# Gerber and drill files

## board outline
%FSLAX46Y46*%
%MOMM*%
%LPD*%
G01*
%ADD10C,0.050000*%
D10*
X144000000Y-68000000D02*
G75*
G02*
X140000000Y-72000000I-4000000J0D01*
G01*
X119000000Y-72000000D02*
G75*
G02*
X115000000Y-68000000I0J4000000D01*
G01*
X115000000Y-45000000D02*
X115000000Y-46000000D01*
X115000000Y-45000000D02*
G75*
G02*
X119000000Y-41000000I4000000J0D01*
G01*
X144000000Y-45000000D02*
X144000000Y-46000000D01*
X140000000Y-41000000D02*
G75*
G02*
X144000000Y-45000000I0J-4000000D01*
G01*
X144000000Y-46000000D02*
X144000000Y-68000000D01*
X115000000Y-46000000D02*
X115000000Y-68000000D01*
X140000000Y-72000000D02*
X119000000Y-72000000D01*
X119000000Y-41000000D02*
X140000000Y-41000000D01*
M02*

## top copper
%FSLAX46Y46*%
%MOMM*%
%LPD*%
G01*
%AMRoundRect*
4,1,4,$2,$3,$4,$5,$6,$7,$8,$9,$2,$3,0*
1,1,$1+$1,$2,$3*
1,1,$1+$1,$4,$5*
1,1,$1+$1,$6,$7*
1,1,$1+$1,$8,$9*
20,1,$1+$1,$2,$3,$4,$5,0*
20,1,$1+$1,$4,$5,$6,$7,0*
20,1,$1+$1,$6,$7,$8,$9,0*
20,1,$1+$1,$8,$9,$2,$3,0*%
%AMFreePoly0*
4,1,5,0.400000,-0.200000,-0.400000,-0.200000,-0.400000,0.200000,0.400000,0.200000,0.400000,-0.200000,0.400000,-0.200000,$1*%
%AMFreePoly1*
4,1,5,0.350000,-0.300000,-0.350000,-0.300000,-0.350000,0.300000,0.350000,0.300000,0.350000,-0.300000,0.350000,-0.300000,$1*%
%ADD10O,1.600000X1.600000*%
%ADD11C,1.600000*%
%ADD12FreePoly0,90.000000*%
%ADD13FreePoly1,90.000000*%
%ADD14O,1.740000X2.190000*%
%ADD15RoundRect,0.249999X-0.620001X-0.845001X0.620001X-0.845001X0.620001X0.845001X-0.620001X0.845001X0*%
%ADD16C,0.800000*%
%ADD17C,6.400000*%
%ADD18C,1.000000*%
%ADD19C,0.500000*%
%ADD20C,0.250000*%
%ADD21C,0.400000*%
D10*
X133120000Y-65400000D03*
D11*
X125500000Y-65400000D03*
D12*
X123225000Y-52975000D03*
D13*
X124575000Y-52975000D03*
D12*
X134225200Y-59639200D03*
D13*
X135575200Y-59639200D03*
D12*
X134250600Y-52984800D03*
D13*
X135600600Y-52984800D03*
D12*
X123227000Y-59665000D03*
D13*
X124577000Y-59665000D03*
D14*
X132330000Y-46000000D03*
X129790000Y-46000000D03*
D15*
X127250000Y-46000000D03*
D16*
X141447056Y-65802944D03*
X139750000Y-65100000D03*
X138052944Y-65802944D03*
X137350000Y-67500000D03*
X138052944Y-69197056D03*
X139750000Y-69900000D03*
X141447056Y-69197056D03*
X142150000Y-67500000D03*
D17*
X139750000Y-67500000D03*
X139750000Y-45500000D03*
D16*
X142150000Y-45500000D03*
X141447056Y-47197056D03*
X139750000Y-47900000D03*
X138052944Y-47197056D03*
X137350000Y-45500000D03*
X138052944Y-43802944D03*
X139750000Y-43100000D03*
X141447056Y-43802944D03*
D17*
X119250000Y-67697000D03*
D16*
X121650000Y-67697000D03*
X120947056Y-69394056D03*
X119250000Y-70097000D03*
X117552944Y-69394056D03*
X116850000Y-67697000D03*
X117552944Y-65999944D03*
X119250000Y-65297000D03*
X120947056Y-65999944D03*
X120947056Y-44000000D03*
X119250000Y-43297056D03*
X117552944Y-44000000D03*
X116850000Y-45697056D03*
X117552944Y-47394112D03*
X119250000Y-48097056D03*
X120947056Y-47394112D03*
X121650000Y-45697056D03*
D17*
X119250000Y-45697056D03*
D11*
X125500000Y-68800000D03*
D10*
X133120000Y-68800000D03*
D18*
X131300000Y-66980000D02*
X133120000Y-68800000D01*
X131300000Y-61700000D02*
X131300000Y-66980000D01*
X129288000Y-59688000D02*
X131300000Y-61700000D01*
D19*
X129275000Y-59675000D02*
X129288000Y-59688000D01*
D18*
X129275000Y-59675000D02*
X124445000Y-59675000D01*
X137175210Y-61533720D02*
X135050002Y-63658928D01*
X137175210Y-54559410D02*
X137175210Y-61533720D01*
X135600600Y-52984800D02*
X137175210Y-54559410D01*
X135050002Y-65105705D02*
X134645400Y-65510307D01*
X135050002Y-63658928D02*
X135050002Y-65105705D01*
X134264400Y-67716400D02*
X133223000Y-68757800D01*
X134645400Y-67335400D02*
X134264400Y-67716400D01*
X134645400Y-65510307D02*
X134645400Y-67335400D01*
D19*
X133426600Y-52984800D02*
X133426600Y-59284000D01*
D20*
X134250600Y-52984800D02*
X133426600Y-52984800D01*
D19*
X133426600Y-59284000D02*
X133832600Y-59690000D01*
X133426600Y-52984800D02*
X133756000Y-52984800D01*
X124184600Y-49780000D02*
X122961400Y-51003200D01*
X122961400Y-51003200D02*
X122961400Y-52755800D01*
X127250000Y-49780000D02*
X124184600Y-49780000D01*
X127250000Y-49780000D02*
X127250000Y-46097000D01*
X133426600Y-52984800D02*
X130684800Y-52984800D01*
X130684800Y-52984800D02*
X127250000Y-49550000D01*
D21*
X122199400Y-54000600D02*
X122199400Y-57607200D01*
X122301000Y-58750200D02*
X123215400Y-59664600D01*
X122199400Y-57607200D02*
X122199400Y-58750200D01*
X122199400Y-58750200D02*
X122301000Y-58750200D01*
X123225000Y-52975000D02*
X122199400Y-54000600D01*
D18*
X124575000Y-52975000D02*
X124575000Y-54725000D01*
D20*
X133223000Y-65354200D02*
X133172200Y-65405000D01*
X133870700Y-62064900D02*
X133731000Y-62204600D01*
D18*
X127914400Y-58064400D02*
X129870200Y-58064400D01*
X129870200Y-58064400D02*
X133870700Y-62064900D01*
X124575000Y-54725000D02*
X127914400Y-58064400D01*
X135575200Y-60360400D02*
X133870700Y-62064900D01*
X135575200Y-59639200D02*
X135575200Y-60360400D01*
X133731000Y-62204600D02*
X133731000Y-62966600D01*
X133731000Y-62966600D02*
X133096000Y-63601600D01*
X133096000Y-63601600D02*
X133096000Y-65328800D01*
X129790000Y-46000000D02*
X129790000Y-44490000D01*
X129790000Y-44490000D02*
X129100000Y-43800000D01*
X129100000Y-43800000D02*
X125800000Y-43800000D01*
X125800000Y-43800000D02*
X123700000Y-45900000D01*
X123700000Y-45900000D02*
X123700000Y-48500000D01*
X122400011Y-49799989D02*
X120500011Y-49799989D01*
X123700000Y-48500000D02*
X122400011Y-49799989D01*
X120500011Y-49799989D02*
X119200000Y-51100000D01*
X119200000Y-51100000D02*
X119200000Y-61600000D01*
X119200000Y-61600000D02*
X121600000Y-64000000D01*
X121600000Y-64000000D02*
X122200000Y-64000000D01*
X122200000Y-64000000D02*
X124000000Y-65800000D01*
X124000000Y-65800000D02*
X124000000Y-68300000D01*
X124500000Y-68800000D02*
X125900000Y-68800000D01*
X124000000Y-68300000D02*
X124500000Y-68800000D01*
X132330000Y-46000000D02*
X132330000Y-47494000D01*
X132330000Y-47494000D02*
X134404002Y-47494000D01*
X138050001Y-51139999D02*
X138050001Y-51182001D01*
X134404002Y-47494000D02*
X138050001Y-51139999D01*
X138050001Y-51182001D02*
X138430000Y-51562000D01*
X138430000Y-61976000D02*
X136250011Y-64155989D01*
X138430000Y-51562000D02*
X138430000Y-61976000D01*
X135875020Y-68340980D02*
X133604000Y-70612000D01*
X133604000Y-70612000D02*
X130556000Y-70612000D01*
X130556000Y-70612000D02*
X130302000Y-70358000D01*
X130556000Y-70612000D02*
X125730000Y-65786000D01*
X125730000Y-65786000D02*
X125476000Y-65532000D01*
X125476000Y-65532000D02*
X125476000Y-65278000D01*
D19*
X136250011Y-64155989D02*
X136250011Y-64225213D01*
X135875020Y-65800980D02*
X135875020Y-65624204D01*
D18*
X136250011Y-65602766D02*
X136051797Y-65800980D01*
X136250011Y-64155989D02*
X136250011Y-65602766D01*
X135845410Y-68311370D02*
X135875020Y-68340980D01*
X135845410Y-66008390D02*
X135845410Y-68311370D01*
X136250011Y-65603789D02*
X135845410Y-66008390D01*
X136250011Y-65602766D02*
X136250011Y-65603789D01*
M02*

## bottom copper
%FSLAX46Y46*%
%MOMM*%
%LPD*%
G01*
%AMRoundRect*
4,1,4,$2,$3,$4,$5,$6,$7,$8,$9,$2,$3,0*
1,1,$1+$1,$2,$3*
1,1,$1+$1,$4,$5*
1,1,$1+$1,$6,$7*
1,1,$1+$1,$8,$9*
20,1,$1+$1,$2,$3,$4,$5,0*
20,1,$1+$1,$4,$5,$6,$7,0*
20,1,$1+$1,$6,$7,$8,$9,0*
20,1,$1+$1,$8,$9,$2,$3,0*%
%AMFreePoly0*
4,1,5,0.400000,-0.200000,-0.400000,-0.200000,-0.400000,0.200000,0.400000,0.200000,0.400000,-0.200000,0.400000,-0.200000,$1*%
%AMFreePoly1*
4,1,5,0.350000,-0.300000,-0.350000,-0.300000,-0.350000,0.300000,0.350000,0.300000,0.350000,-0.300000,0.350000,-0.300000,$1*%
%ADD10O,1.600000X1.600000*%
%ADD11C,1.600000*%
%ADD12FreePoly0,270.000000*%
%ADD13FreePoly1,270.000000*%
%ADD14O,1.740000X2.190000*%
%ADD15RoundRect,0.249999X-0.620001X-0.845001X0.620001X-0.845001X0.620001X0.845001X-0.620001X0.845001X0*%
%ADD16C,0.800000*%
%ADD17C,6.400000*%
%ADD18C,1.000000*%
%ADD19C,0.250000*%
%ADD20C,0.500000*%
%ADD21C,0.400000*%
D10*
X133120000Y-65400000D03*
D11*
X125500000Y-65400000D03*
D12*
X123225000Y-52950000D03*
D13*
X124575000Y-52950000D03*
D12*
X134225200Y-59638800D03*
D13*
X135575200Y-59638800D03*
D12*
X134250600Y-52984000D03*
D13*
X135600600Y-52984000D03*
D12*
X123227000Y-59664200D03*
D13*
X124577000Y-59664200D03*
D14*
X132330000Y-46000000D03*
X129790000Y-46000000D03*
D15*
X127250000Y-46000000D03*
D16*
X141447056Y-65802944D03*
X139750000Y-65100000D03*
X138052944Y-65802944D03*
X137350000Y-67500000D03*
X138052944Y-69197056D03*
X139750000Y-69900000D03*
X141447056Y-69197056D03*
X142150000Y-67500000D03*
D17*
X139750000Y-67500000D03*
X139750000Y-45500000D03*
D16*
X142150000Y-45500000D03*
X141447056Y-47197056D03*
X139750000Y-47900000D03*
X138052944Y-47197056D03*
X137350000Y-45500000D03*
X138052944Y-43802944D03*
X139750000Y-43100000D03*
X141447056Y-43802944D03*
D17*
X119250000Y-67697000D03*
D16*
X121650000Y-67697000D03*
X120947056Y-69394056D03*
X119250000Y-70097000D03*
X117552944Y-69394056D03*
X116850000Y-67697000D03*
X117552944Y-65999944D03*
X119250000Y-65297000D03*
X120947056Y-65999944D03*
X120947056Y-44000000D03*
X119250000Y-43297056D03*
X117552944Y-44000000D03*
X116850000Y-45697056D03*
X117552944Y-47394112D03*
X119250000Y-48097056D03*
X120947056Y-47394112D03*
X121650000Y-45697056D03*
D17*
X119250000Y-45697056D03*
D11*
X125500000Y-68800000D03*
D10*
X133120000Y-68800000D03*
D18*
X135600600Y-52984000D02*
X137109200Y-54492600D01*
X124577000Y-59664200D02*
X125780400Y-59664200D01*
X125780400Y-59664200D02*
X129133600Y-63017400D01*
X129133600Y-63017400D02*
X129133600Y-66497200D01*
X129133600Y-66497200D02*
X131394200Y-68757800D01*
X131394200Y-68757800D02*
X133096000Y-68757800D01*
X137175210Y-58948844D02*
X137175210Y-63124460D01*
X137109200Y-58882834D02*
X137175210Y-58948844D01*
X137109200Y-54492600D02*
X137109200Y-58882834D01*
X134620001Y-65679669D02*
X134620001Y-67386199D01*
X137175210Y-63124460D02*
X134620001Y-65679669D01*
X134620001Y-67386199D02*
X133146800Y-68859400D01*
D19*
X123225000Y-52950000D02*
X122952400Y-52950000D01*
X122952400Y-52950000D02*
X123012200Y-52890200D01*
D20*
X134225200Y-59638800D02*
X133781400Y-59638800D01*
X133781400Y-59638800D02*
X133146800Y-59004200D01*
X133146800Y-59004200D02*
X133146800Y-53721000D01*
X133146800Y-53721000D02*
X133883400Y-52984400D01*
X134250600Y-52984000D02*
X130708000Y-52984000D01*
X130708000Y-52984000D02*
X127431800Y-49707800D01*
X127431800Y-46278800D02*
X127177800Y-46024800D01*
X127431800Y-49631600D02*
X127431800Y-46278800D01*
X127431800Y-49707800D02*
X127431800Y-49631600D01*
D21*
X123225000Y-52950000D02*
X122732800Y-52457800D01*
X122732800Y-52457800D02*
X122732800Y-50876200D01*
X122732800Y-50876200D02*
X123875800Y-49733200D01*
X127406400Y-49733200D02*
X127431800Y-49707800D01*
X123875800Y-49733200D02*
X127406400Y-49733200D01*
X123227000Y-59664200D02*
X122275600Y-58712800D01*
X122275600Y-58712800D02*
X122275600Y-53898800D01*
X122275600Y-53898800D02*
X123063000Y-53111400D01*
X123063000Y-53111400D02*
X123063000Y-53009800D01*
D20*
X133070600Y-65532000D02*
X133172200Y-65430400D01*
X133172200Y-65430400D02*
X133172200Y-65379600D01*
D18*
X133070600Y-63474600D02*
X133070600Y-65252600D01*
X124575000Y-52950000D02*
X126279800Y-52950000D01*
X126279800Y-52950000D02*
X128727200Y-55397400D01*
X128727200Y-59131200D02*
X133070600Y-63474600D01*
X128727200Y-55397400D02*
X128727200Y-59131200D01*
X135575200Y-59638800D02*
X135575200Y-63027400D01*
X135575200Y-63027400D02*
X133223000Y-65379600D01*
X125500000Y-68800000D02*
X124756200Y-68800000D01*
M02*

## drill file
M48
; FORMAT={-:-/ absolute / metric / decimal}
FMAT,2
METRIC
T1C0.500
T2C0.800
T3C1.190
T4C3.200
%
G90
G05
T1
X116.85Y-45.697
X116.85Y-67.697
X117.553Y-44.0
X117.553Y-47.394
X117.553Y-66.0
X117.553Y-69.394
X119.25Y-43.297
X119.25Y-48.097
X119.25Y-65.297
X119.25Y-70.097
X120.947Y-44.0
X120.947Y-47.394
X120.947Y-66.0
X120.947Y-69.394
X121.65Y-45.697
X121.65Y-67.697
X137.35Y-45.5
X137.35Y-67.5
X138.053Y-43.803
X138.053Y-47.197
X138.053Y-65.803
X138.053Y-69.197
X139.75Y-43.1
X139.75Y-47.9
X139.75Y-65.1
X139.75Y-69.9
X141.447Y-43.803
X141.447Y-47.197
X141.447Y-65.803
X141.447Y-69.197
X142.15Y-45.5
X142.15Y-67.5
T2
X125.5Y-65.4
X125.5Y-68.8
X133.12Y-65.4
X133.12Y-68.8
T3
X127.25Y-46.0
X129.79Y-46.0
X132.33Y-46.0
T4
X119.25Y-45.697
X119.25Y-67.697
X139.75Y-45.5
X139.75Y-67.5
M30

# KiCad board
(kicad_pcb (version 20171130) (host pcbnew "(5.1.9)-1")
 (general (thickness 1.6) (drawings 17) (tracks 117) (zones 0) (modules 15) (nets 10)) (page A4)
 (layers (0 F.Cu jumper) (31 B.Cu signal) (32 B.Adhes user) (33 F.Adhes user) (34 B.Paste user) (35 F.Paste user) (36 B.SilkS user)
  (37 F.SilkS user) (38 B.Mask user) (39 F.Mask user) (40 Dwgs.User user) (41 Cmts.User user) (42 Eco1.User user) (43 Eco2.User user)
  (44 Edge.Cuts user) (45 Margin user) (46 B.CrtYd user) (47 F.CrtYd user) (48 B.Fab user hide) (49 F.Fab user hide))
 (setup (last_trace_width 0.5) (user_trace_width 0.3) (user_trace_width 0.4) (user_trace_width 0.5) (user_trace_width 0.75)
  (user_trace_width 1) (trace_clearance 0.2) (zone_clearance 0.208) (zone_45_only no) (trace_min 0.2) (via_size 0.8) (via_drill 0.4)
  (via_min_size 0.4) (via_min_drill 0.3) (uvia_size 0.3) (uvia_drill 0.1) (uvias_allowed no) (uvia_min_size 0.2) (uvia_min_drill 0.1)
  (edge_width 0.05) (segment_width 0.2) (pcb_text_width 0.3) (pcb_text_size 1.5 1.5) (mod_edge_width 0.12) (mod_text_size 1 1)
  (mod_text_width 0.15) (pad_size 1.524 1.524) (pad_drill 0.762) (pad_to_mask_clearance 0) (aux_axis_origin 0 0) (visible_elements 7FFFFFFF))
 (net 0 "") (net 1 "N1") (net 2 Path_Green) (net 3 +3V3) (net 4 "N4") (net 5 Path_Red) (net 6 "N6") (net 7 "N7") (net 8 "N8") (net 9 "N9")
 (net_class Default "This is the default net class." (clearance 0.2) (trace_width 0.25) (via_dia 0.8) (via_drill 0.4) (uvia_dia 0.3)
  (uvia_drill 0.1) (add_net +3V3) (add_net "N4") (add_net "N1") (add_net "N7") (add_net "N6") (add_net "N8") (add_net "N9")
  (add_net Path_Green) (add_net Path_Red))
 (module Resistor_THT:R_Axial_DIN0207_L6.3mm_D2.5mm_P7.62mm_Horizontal (layer F.Cu) (at 125.5 65.4)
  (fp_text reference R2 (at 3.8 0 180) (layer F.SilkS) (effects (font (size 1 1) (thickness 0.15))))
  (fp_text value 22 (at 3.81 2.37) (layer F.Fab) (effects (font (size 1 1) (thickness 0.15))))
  (pad 2 thru_hole oval (at 7.62 0) (size 1.6 1.6) (drill 0.8) (layers *.Cu *.Mask) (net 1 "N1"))
  (pad 1 thru_hole circle (at 0 0) (size 1.6 1.6) (drill 0.8) (layers *.Cu *.Mask) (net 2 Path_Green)))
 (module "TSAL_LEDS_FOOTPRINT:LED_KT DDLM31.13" (layer F.Cu) (at 123.95 53 90)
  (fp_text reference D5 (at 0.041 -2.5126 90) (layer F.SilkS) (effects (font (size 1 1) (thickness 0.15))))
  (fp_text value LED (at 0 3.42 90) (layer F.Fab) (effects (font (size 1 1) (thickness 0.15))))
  (pad 2 smd custom (at 0.025 -0.725 90) (size 0.8 0.4) (layers F.Cu F.Paste F.Mask) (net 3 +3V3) (zone_connect 0)
   (options (clearance outline) (anchor rect)) (primitives))
  (pad 1 smd custom (at 0.025 0.625 90) (size 0.7 0.6) (layers F.Cu F.Paste F.Mask) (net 1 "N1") (zone_connect 0)
   (options (clearance outline) (anchor rect)) (primitives)))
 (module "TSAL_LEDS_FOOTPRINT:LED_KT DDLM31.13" (layer B.Cu) (at 123.95 52.925 270)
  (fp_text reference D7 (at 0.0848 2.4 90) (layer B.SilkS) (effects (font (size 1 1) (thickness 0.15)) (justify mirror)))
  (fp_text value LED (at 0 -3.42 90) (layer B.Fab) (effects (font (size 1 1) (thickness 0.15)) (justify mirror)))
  (pad 2 smd custom (at 0.025 0.725 270) (size 0.8 0.4) (layers B.Cu B.Paste B.Mask) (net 3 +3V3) (zone_connect 0)
   (options (clearance outline) (anchor rect)) (primitives))
  (pad 1 smd custom (at 0.025 -0.625 270) (size 0.7 0.6) (layers B.Cu B.Paste B.Mask) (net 1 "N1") (zone_connect 0)
   (options (clearance outline) (anchor rect)) (primitives)))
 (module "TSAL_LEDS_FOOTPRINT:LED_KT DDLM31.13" (layer B.Cu) (at 134.9502 59.6138 270)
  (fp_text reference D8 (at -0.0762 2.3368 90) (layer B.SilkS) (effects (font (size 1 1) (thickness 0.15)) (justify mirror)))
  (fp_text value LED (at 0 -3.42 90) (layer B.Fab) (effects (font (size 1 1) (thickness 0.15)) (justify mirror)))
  (pad 2 smd custom (at 0.025 0.725 270) (size 0.8 0.4) (layers B.Cu B.Paste B.Mask) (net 3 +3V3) (zone_connect 0)
   (options (clearance outline) (anchor rect)) (primitives))
  (pad 1 smd custom (at 0.025 -0.625 270) (size 0.7 0.6) (layers B.Cu B.Paste B.Mask) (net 1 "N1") (zone_connect 0)
   (options (clearance outline) (anchor rect)) (primitives)))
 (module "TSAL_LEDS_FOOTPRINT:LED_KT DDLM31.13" (layer F.Cu) (at 134.9502 59.6642 90)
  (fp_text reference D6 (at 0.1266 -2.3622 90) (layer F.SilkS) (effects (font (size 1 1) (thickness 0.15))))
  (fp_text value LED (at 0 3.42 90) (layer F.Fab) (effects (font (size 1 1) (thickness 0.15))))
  (pad 2 smd custom (at 0.025 -0.725 90) (size 0.8 0.4) (layers F.Cu F.Paste F.Mask) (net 3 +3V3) (zone_connect 0)
   (options (clearance outline) (anchor rect)) (primitives))
  (pad 1 smd custom (at 0.025 0.625 90) (size 0.7 0.6) (layers F.Cu F.Paste F.Mask) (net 1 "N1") (zone_connect 0)
   (options (clearance outline) (anchor rect)) (primitives)))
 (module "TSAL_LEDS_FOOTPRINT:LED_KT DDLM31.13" (layer B.Cu) (at 134.9756 52.959 270)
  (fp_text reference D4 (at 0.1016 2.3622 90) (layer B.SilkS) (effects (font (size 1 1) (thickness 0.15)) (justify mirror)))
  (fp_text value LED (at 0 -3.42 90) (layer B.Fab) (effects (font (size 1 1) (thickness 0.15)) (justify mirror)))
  (pad 2 smd custom (at 0.025 0.725 270) (size 0.8 0.4) (layers B.Cu B.Paste B.Mask) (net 3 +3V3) (zone_connect 0)
   (options (clearance outline) (anchor rect)) (primitives))
  (pad 1 smd custom (at 0.025 -0.625 270) (size 0.7 0.6) (layers B.Cu B.Paste B.Mask) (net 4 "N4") (zone_connect 0)
   (options (clearance outline) (anchor rect)) (primitives)))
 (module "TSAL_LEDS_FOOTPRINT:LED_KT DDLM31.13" (layer B.Cu) (at 123.952 59.6392 270)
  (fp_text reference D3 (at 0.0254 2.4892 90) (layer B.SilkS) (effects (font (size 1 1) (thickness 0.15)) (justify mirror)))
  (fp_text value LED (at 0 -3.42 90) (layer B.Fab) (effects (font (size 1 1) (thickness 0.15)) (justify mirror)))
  (pad 2 smd custom (at 0.025 0.725 270) (size 0.8 0.4) (layers B.Cu B.Paste B.Mask) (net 3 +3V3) (zone_connect 0)
   (options (clearance outline) (anchor rect)) (primitives))
  (pad 1 smd custom (at 0.025 -0.625 270) (size 0.7 0.6) (layers B.Cu B.Paste B.Mask) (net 4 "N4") (zone_connect 0)
   (options (clearance outline) (anchor rect)) (primitives)))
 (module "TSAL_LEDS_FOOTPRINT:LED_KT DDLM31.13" (layer F.Cu) (at 134.9756 53.0098 90)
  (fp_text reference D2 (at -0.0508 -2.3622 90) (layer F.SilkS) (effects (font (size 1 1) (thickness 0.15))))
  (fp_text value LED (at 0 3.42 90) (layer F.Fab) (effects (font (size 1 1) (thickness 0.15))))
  (pad 2 smd custom (at 0.025 -0.725 90) (size 0.8 0.4) (layers F.Cu F.Paste F.Mask) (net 3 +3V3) (zone_connect 0)
   (options (clearance outline) (anchor rect)) (primitives))
  (pad 1 smd custom (at 0.025 0.625 90) (size 0.7 0.6) (layers F.Cu F.Paste F.Mask) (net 4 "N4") (zone_connect 0)
   (options (clearance outline) (anchor rect)) (primitives)))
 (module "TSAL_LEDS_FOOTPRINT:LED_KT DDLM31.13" (layer F.Cu) (at 123.952 59.69 90)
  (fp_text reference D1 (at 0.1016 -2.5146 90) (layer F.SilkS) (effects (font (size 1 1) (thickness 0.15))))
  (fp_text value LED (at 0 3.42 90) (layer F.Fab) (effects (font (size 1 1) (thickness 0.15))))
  (pad 2 smd custom (at 0.025 -0.725 90) (size 0.8 0.4) (layers F.Cu F.Paste F.Mask) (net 3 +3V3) (zone_connect 0)
   (options (clearance outline) (anchor rect)) (primitives))
  (pad 1 smd custom (at 0.025 0.625 90) (size 0.7 0.6) (layers F.Cu F.Paste F.Mask) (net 4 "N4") (zone_connect 0)
   (options (clearance outline) (anchor rect)) (primitives)))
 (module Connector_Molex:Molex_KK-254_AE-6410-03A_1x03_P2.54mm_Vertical (layer F.Cu) (at 127.25 46)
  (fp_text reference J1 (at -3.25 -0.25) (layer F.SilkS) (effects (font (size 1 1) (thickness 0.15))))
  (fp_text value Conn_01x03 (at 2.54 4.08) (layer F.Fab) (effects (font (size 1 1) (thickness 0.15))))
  (pad 3 thru_hole oval (at 5.08 0) (size 1.74 2.19) (drill 1.19) (layers *.Cu *.Mask) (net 2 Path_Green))
  (pad 2 thru_hole oval (at 2.54 0) (size 1.74 2.19) (drill 1.19) (layers *.Cu *.Mask) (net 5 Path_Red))
  (pad 1 thru_hole roundrect (at 0 0) (size 1.74 2.19) (drill 1.19) (layers *.Cu *.Mask) (roundrect_rratio 0.1436775862068966) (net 3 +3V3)))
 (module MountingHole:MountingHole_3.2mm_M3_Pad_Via (layer F.Cu) (at 139.75 67.5)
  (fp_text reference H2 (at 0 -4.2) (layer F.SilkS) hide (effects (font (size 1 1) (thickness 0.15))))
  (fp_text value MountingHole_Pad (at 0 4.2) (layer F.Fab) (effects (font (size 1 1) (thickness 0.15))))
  (pad 1 thru_hole circle (at 1.697056 -1.697056) (size 0.8 0.8) (drill 0.5) (layers *.Cu *.Mask) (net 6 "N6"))
  (pad 1 thru_hole circle (at 0 -2.4) (size 0.8 0.8) (drill 0.5) (layers *.Cu *.Mask) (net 6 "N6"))
  (pad 1 thru_hole circle (at -1.697056 -1.697056) (size 0.8 0.8) (drill 0.5) (layers *.Cu *.Mask) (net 6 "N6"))
  (pad 1 thru_hole circle (at -2.4 0) (size 0.8 0.8) (drill 0.5) (layers *.Cu *.Mask) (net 6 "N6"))
  (pad 1 thru_hole circle (at -1.697056 1.697056) (size 0.8 0.8) (drill 0.5) (layers *.Cu *.Mask) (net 6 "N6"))
  (pad 1 thru_hole circle (at 0 2.4) (size 0.8 0.8) (drill 0.5) (layers *.Cu *.Mask) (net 6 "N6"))
  (pad 1 thru_hole circle (at 1.697056 1.697056) (size 0.8 0.8) (drill 0.5) (layers *.Cu *.Mask) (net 6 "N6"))
  (pad 1 thru_hole circle (at 2.4 0) (size 0.8 0.8) (drill 0.5) (layers *.Cu *.Mask) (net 6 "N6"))
  (pad 1 thru_hole circle (at 0 0) (size 6.4 6.4) (drill 3.2) (layers *.Cu *.Mask) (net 6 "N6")))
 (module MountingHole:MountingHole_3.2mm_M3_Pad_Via (layer F.Cu) (at 139.75 45.5)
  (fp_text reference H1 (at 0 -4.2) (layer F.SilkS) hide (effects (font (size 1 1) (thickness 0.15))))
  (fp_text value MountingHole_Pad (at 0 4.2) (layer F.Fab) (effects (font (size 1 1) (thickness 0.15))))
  (pad 1 thru_hole circle (at 0 0) (size 6.4 6.4) (drill 3.2) (layers *.Cu *.Mask) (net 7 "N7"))
  (pad 1 thru_hole circle (at 2.4 0) (size 0.8 0.8) (drill 0.5) (layers *.Cu *.Mask) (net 7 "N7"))
  (pad 1 thru_hole circle (at 1.697056 1.697056) (size 0.8 0.8) (drill 0.5) (layers *.Cu *.Mask) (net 7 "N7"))
  (pad 1 thru_hole circle (at 0 2.4) (size 0.8 0.8) (drill 0.5) (layers *.Cu *.Mask) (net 7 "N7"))
  (pad 1 thru_hole circle (at -1.697056 1.697056) (size 0.8 0.8) (drill 0.5) (layers *.Cu *.Mask) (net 7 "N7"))
  (pad 1 thru_hole circle (at -2.4 0) (size 0.8 0.8) (drill 0.5) (layers *.Cu *.Mask) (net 7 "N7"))
  (pad 1 thru_hole circle (at -1.697056 -1.697056) (size 0.8 0.8) (drill 0.5) (layers *.Cu *.Mask) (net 7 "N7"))
  (pad 1 thru_hole circle (at 0 -2.4) (size 0.8 0.8) (drill 0.5) (layers *.Cu *.Mask) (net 7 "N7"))
  (pad 1 thru_hole circle (at 1.697056 -1.697056) (size 0.8 0.8) (drill 0.5) (layers *.Cu *.Mask) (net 7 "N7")))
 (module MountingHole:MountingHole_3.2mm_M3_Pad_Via (layer F.Cu) (at 119.25 67.697)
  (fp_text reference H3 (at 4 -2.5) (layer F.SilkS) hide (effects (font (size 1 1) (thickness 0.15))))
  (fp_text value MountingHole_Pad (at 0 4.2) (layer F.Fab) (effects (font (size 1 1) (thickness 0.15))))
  (pad 1 thru_hole circle (at 0 0) (size 6.4 6.4) (drill 3.2) (layers *.Cu *.Mask) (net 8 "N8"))
  (pad 1 thru_hole circle (at 2.4 0) (size 0.8 0.8) (drill 0.5) (layers *.Cu *.Mask) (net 8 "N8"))
  (pad 1 thru_hole circle (at 1.697056 1.697056) (size 0.8 0.8) (drill 0.5) (layers *.Cu *.Mask) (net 8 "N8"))
  (pad 1 thru_hole circle (at 0 2.4) (size 0.8 0.8) (drill 0.5) (layers *.Cu *.Mask) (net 8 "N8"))
  (pad 1 thru_hole circle (at -1.697056 1.697056) (size 0.8 0.8) (drill 0.5) (layers *.Cu *.Mask) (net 8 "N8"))
  (pad 1 thru_hole circle (at -2.4 0) (size 0.8 0.8) (drill 0.5) (layers *.Cu *.Mask) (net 8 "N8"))
  (pad 1 thru_hole circle (at -1.697056 -1.697056) (size 0.8 0.8) (drill 0.5) (layers *.Cu *.Mask) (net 8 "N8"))
  (pad 1 thru_hole circle (at 0 -2.4) (size 0.8 0.8) (drill 0.5) (layers *.Cu *.Mask) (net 8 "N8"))
  (pad 1 thru_hole circle (at 1.697056 -1.697056) (size 0.8 0.8) (drill 0.5) (layers *.Cu *.Mask) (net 8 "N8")))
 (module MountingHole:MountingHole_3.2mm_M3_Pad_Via (layer F.Cu) (at 119.25 45.697056)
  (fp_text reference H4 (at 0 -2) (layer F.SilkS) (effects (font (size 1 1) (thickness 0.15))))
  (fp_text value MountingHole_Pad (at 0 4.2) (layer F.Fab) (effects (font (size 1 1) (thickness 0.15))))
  (pad 1 thru_hole circle (at 1.697056 -1.697056) (size 0.8 0.8) (drill 0.5) (layers *.Cu *.Mask) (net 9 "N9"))
  (pad 1 thru_hole circle (at 0 -2.4) (size 0.8 0.8) (drill 0.5) (layers *.Cu *.Mask) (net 9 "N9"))
  (pad 1 thru_hole circle (at -1.697056 -1.697056) (size 0.8 0.8) (drill 0.5) (layers *.Cu *.Mask) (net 9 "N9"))
  (pad 1 thru_hole circle (at -2.4 0) (size 0.8 0.8) (drill 0.5) (layers *.Cu *.Mask) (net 9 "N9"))
  (pad 1 thru_hole circle (at -1.697056 1.697056) (size 0.8 0.8) (drill 0.5) (layers *.Cu *.Mask) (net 9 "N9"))
  (pad 1 thru_hole circle (at 0 2.4) (size 0.8 0.8) (drill 0.5) (layers *.Cu *.Mask) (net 9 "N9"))
  (pad 1 thru_hole circle (at 1.697056 1.697056) (size 0.8 0.8) (drill 0.5) (layers *.Cu *.Mask) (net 9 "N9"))
  (pad 1 thru_hole circle (at 2.4 0) (size 0.8 0.8) (drill 0.5) (layers *.Cu *.Mask) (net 9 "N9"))
  (pad 1 thru_hole circle (at 0 0) (size 6.4 6.4) (drill 3.2) (layers *.Cu *.Mask) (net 9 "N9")))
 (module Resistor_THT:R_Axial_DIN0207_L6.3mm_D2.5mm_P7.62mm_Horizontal (layer F.Cu) (at 125.5 68.8)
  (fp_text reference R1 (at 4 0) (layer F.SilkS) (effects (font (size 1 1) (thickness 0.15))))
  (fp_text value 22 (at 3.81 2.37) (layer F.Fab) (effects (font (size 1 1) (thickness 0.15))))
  (pad 1 thru_hole circle (at 0 0) (size 1.6 1.6) (drill 0.8) (layers *.Cu *.Mask) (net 5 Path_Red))
  (pad 2 thru_hole oval (at 7.62 0) (size 1.6 1.6) (drill 0.8) (layers *.Cu *.Mask) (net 4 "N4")))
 (gr_arc (start 140 68) (end 140 72) (angle -90) (layer Edge.Cuts) (width 0.05))
 (gr_arc (start 119 68) (end 115 68) (angle -90) (layer Edge.Cuts) (width 0.05))
 (gr_line (start 115 45) (end 115 46) (layer Edge.Cuts) (width 0.05))
 (gr_arc (start 119 45) (end 119 41) (angle -90) (layer Edge.Cuts) (width 0.05))
 (gr_line (start 144 45) (end 144 46) (layer Edge.Cuts) (width 0.05))
 (gr_arc (start 140 45) (end 144 45) (angle -90) (layer Edge.Cuts) (width 0.05))
 (gr_line (start 144 46) (end 144 68) (layer Edge.Cuts) (width 0.05))
 (gr_line (start 115 46) (end 115 68) (layer Edge.Cuts) (width 0.05))
 (gr_line (start 140 72) (end 119 72) (layer Edge.Cuts) (width 0.05))
 (gr_line (start 119 41) (end 140 41) (layer Edge.Cuts) (width 0.05))
 (segment (start 131.3 66.98) (end 133.12 68.8) (width 1) (layer F.Cu) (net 4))
 (segment (start 131.3 61.7) (end 131.3 66.98) (width 1) (layer F.Cu) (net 4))
 (segment (start 129.288 59.688) (end 131.3 61.7) (width 1) (layer F.Cu) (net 4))
 (segment (start 129.275 59.675) (end 129.288 59.688) (width 0.5) (layer F.Cu) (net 4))
 (segment (start 129.275 59.675) (end 124.445 59.675) (width 1) (layer F.Cu) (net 4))
 (segment (start 137.17521 61.53372) (end 135.050002 63.658928) (width 1) (layer F.Cu) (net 4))
 (segment (start 137.17521 54.55941) (end 137.17521 61.53372) (width 1) (layer F.Cu) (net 4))
 (segment (start 135.6006 52.9848) (end 137.17521 54.55941) (width 1) (layer F.Cu) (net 4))
 (segment (start 135.050002 65.105705) (end 134.6454 65.510307) (width 1) (layer F.Cu) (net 4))
 (segment (start 135.050002 63.658928) (end 135.050002 65.105705) (width 1) (layer F.Cu) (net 4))
 (segment (start 134.2644 67.7164) (end 133.223 68.7578) (width 1) (layer F.Cu) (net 4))
 (segment (start 135.6006 52.984) (end 137.1092 54.4926) (width 1) (layer B.Cu) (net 4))
 (segment (start 124.577 59.6642) (end 125.7804 59.6642) (width 1) (layer B.Cu) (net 4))
 (segment (start 125.7804 59.6642) (end 129.1336 63.0174) (width 1) (layer B.Cu) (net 4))
 (segment (start 129.1336 63.0174) (end 129.1336 66.4972) (width 1) (layer B.Cu) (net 4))
 (segment (start 129.1336 66.4972) (end 131.3942 68.7578) (width 1) (layer B.Cu) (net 4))
 (segment (start 131.3942 68.7578) (end 133.096 68.7578) (width 1) (layer B.Cu) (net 4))
 (segment (start 134.6454 67.3354) (end 134.2644 67.7164) (width 1) (layer F.Cu) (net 4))
 (segment (start 134.6454 65.510307) (end 134.6454 67.3354) (width 1) (layer F.Cu) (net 4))
 (segment (start 137.17521 58.948844) (end 137.17521 63.12446) (width 1) (layer B.Cu) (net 4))
 (segment (start 137.1092 58.882834) (end 137.17521 58.948844) (width 1) (layer B.Cu) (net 4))
 (segment (start 137.1092 54.4926) (end 137.1092 58.882834) (width 1) (layer B.Cu) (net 4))
 (segment (start 134.620001 65.679669) (end 134.620001 67.386199) (width 1) (layer B.Cu) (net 4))
 (segment (start 137.17521 63.12446) (end 134.620001 65.679669) (width 1) (layer B.Cu) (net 4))
 (segment (start 134.620001 67.386199) (end 133.1468 68.8594) (width 1) (layer B.Cu) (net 4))
 (segment (start 123.225 52.95) (end 122.9524 52.95) (width 0.25) (layer B.Cu) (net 3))
 (segment (start 122.9524 52.95) (end 123.0122 52.8902) (width 0.25) (layer B.Cu) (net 3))
 (segment (start 133.4266 52.9848) (end 133.4266 59.284) (width 0.5) (layer F.Cu) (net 3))
 (segment (start 134.2506 52.9848) (end 133.4266 52.9848) (width 0.25) (layer F.Cu) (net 3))
 (segment (start 133.4266 59.284) (end 133.8326 59.69) (width 0.5) (layer F.Cu) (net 3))
 (segment (start 133.4266 52.9848) (end 133.756 52.9848) (width 0.5) (layer F.Cu) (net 3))
 (segment (start 124.1846 49.78) (end 122.9614 51.0032) (width 0.5) (layer F.Cu) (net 3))
 (segment (start 122.9614 51.0032) (end 122.9614 52.7558) (width 0.5) (layer F.Cu) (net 3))
 (segment (start 127.25 49.78) (end 124.1846 49.78) (width 0.5) (layer F.Cu) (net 3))
 (segment (start 127.25 49.78) (end 127.25 46.097) (width 0.5) (layer F.Cu) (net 3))
 (segment (start 134.2252 59.6388) (end 133.7814 59.6388) (width 0.5) (layer B.Cu) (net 3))
 (segment (start 133.7814 59.6388) (end 133.1468 59.0042) (width 0.5) (layer B.Cu) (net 3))
 (segment (start 133.1468 59.0042) (end 133.1468 53.721) (width 0.5) (layer B.Cu) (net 3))
 (segment (start 133.1468 53.721) (end 133.8834 52.9844) (width 0.5) (layer B.Cu) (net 3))
 (segment (start 133.4266 52.9848) (end 130.6848 52.9848) (width 0.5) (layer F.Cu) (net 3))
 (segment (start 130.6848 52.9848) (end 127.25 49.55) (width 0.5) (layer F.Cu) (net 3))
 (segment (start 134.2506 52.984) (end 130.708 52.984) (width 0.5) (layer B.Cu) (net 3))
 (segment (start 130.708 52.984) (end 127.4318 49.7078) (width 0.5) (layer B.Cu) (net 3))
 (segment (start 127.4318 46.2788) (end 127.1778 46.0248) (width 0.5) (layer B.Cu) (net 3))
 (segment (start 127.4318 49.6316) (end 127.4318 46.2788) (width 0.5) (layer B.Cu) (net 3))
 (segment (start 127.4318 49.7078) (end 127.4318 49.6316) (width 0.5) (layer B.Cu) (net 3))
 (segment (start 123.225 52.95) (end 122.7328 52.4578) (width 0.4) (layer B.Cu) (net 3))
 (segment (start 122.7328 52.4578) (end 122.7328 50.8762) (width 0.4) (layer B.Cu) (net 3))
 (segment (start 122.7328 50.8762) (end 123.8758 49.7332) (width 0.4) (layer B.Cu) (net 3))
 (segment (start 127.4064 49.7332) (end 127.4318 49.7078) (width 0.4) (layer B.Cu) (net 3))
 (segment (start 123.8758 49.7332) (end 127.4064 49.7332) (width 0.4) (layer B.Cu) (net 3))
 (segment (start 122.1994 54.0006) (end 122.1994 57.6072) (width 0.4) (layer F.Cu) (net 3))
 (segment (start 122.301 58.7502) (end 123.2154 59.6646) (width 0.4) (layer F.Cu) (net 3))
 (segment (start 122.1994 57.6072) (end 122.1994 58.7502) (width 0.4) (layer F.Cu) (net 3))
 (segment (start 122.1994 58.7502) (end 122.301 58.7502) (width 0.4) (layer F.Cu) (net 3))
 (segment (start 123.225 52.975) (end 122.1994 54.0006) (width 0.4) (layer F.Cu) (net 3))
 (segment (start 123.227 59.6642) (end 122.2756 58.7128) (width 0.4) (layer B.Cu) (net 3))
 (segment (start 122.2756 58.7128) (end 122.2756 53.8988) (width 0.4) (layer B.Cu) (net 3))
 (segment (start 122.2756 53.8988) (end 123.063 53.1114) (width 0.4) (layer B.Cu) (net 3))
 (segment (start 123.063 53.1114) (end 123.063 53.0098) (width 0.4) (layer B.Cu) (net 3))
 (segment (start 133.0706 65.532) (end 133.1722 65.4304) (width 0.5) (layer B.Cu) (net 1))
 (segment (start 133.1722 65.4304) (end 133.1722 65.3796) (width 0.5) (layer B.Cu) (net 1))
 (segment (start 124.575 52.975) (end 124.575 54.725) (width 1) (layer F.Cu) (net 1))
 (segment (start 133.223 65.3542) (end 133.1722 65.405) (width 0.25) (layer F.Cu) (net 1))
 (segment (start 133.8707 62.0649) (end 133.731 62.2046) (width 0.25) (layer F.Cu) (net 1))
 (segment (start 127.9144 58.0644) (end 129.8702 58.0644) (width 1) (layer F.Cu) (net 1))
 (segment (start 129.8702 58.0644) (end 133.8707 62.0649) (width 1) (layer F.Cu) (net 1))
 (segment (start 124.575 54.725) (end 127.9144 58.0644) (width 1) (layer F.Cu) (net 1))
 (segment (start 135.5752 60.3604) (end 133.8707 62.0649) (width 1) (layer F.Cu) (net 1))
 (segment (start 135.5752 59.6392) (end 135.5752 60.3604) (width 1) (layer F.Cu) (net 1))
 (segment (start 133.731 62.2046) (end 133.731 62.9666) (width 1) (layer F.Cu) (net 1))
 (segment (start 133.731 62.9666) (end 133.096 63.6016) (width 1) (layer F.Cu) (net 1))
 (segment (start 133.096 63.6016) (end 133.096 65.3288) (width 1) (layer F.Cu) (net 1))
 (segment (start 133.0706 63.4746) (end 133.0706 65.2526) (width 1) (layer B.Cu) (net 1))
 (segment (start 124.575 52.95) (end 126.2798 52.95) (width 1) (layer B.Cu) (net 1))
 (segment (start 126.2798 52.95) (end 128.7272 55.3974) (width 1) (layer B.Cu) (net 1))
 (segment (start 128.7272 59.1312) (end 133.0706 63.4746) (width 1) (layer B.Cu) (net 1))
 (segment (start 128.7272 55.3974) (end 128.7272 59.1312) (width 1) (layer B.Cu) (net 1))
 (segment (start 135.5752 59.6388) (end 135.5752 63.0274) (width 1) (layer B.Cu) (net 1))
 (segment (start 135.5752 63.0274) (end 133.223 65.3796) (width 1) (layer B.Cu) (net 1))
 (segment (start 129.79 46) (end 129.79 44.49) (width 1) (layer F.Cu) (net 5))
 (segment (start 129.79 44.49) (end 129.1 43.8) (width 1) (layer F.Cu) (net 5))
 (segment (start 129.1 43.8) (end 125.8 43.8) (width 1) (layer F.Cu) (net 5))
 (segment (start 125.8 43.8) (end 123.7 45.9) (width 1) (layer F.Cu) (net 5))
 (segment (start 123.7 45.9) (end 123.7 48.5) (width 1) (layer F.Cu) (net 5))
 (segment (start 122.400011 49.799989) (end 120.500011 49.799989) (width 1) (layer F.Cu) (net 5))
 (segment (start 123.7 48.5) (end 122.400011 49.799989) (width 1) (layer F.Cu) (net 5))
 (segment (start 120.500011 49.799989) (end 119.2 51.1) (width 1) (layer F.Cu) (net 5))
 (segment (start 119.2 51.1) (end 119.2 61.6) (width 1) (layer F.Cu) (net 5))
 (segment (start 119.2 61.6) (end 121.6 64) (width 1) (layer F.Cu) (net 5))
 (segment (start 121.6 64) (end 122.2 64) (width 1) (layer F.Cu) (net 5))
 (segment (start 122.2 64) (end 124 65.8) (width 1) (layer F.Cu) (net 5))
 (segment (start 124 65.8) (end 124 68.3) (width 1) (layer F.Cu) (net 5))
 (segment (start 124.5 68.8) (end 125.9 68.8) (width 1) (layer F.Cu) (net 5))
 (segment (start 124 68.3) (end 124.5 68.8) (width 1) (layer F.Cu) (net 5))
 (segment (start 125.5 68.8) (end 124.7562 68.8) (width 1) (layer B.Cu) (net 5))
 (segment (start 132.33 46) (end 132.33 47.494) (width 1) (layer F.Cu) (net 2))
 (segment (start 132.33 47.494) (end 134.404002 47.494) (width 1) (layer F.Cu) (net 2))
 (segment (start 138.050001 51.139999) (end 138.050001 51.182001) (width 1) (layer F.Cu) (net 2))
 (segment (start 134.404002 47.494) (end 138.050001 51.139999) (width 1) (layer F.Cu) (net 2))
 (segment (start 138.050001 51.182001) (end 138.43 51.562) (width 1) (layer F.Cu) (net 2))
 (segment (start 138.43 61.976) (end 136.250011 64.155989) (width 1) (layer F.Cu) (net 2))
 (segment (start 138.43 51.562) (end 138.43 61.976) (width 1) (layer F.Cu) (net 2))
 (segment (start 135.87502 68.34098) (end 133.604 70.612) (width 1) (layer F.Cu) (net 2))
 (segment (start 133.604 70.612) (end 130.556 70.612) (width 1) (layer F.Cu) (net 2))
 (segment (start 130.556 70.612) (end 130.302 70.358) (width 1) (layer F.Cu) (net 2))
 (segment (start 130.556 70.612) (end 125.73 65.786) (width 1) (layer F.Cu) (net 2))
 (segment (start 125.73 65.786) (end 125.476 65.532) (width 1) (layer F.Cu) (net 2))
 (segment (start 125.476 65.532) (end 125.476 65.278) (width 1) (layer F.Cu) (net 2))
 (segment (start 136.250011 64.155989) (end 136.250011 64.225213) (width 0.5) (layer F.Cu) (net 2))
 (segment (start 135.87502 65.80098) (end 135.87502 65.624204) (width 0.5) (layer F.Cu) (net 2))
 (segment (start 136.250011 65.602766) (end 136.051797 65.80098) (width 1) (layer F.Cu) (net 2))
 (segment (start 136.250011 64.155989) (end 136.250011 65.602766) (width 1) (layer F.Cu) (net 2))
 (segment (start 135.84541 68.31137) (end 135.87502 68.34098) (width 1) (layer F.Cu) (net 2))
 (segment (start 135.84541 66.00839) (end 135.84541 68.31137) (width 1) (layer F.Cu) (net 2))
 (segment (start 136.250011 65.603789) (end 135.84541 66.00839) (width 1) (layer F.Cu) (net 2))
 (segment (start 136.250011 65.602766) (end 136.250011 65.603789) (width 1) (layer F.Cu) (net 2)))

